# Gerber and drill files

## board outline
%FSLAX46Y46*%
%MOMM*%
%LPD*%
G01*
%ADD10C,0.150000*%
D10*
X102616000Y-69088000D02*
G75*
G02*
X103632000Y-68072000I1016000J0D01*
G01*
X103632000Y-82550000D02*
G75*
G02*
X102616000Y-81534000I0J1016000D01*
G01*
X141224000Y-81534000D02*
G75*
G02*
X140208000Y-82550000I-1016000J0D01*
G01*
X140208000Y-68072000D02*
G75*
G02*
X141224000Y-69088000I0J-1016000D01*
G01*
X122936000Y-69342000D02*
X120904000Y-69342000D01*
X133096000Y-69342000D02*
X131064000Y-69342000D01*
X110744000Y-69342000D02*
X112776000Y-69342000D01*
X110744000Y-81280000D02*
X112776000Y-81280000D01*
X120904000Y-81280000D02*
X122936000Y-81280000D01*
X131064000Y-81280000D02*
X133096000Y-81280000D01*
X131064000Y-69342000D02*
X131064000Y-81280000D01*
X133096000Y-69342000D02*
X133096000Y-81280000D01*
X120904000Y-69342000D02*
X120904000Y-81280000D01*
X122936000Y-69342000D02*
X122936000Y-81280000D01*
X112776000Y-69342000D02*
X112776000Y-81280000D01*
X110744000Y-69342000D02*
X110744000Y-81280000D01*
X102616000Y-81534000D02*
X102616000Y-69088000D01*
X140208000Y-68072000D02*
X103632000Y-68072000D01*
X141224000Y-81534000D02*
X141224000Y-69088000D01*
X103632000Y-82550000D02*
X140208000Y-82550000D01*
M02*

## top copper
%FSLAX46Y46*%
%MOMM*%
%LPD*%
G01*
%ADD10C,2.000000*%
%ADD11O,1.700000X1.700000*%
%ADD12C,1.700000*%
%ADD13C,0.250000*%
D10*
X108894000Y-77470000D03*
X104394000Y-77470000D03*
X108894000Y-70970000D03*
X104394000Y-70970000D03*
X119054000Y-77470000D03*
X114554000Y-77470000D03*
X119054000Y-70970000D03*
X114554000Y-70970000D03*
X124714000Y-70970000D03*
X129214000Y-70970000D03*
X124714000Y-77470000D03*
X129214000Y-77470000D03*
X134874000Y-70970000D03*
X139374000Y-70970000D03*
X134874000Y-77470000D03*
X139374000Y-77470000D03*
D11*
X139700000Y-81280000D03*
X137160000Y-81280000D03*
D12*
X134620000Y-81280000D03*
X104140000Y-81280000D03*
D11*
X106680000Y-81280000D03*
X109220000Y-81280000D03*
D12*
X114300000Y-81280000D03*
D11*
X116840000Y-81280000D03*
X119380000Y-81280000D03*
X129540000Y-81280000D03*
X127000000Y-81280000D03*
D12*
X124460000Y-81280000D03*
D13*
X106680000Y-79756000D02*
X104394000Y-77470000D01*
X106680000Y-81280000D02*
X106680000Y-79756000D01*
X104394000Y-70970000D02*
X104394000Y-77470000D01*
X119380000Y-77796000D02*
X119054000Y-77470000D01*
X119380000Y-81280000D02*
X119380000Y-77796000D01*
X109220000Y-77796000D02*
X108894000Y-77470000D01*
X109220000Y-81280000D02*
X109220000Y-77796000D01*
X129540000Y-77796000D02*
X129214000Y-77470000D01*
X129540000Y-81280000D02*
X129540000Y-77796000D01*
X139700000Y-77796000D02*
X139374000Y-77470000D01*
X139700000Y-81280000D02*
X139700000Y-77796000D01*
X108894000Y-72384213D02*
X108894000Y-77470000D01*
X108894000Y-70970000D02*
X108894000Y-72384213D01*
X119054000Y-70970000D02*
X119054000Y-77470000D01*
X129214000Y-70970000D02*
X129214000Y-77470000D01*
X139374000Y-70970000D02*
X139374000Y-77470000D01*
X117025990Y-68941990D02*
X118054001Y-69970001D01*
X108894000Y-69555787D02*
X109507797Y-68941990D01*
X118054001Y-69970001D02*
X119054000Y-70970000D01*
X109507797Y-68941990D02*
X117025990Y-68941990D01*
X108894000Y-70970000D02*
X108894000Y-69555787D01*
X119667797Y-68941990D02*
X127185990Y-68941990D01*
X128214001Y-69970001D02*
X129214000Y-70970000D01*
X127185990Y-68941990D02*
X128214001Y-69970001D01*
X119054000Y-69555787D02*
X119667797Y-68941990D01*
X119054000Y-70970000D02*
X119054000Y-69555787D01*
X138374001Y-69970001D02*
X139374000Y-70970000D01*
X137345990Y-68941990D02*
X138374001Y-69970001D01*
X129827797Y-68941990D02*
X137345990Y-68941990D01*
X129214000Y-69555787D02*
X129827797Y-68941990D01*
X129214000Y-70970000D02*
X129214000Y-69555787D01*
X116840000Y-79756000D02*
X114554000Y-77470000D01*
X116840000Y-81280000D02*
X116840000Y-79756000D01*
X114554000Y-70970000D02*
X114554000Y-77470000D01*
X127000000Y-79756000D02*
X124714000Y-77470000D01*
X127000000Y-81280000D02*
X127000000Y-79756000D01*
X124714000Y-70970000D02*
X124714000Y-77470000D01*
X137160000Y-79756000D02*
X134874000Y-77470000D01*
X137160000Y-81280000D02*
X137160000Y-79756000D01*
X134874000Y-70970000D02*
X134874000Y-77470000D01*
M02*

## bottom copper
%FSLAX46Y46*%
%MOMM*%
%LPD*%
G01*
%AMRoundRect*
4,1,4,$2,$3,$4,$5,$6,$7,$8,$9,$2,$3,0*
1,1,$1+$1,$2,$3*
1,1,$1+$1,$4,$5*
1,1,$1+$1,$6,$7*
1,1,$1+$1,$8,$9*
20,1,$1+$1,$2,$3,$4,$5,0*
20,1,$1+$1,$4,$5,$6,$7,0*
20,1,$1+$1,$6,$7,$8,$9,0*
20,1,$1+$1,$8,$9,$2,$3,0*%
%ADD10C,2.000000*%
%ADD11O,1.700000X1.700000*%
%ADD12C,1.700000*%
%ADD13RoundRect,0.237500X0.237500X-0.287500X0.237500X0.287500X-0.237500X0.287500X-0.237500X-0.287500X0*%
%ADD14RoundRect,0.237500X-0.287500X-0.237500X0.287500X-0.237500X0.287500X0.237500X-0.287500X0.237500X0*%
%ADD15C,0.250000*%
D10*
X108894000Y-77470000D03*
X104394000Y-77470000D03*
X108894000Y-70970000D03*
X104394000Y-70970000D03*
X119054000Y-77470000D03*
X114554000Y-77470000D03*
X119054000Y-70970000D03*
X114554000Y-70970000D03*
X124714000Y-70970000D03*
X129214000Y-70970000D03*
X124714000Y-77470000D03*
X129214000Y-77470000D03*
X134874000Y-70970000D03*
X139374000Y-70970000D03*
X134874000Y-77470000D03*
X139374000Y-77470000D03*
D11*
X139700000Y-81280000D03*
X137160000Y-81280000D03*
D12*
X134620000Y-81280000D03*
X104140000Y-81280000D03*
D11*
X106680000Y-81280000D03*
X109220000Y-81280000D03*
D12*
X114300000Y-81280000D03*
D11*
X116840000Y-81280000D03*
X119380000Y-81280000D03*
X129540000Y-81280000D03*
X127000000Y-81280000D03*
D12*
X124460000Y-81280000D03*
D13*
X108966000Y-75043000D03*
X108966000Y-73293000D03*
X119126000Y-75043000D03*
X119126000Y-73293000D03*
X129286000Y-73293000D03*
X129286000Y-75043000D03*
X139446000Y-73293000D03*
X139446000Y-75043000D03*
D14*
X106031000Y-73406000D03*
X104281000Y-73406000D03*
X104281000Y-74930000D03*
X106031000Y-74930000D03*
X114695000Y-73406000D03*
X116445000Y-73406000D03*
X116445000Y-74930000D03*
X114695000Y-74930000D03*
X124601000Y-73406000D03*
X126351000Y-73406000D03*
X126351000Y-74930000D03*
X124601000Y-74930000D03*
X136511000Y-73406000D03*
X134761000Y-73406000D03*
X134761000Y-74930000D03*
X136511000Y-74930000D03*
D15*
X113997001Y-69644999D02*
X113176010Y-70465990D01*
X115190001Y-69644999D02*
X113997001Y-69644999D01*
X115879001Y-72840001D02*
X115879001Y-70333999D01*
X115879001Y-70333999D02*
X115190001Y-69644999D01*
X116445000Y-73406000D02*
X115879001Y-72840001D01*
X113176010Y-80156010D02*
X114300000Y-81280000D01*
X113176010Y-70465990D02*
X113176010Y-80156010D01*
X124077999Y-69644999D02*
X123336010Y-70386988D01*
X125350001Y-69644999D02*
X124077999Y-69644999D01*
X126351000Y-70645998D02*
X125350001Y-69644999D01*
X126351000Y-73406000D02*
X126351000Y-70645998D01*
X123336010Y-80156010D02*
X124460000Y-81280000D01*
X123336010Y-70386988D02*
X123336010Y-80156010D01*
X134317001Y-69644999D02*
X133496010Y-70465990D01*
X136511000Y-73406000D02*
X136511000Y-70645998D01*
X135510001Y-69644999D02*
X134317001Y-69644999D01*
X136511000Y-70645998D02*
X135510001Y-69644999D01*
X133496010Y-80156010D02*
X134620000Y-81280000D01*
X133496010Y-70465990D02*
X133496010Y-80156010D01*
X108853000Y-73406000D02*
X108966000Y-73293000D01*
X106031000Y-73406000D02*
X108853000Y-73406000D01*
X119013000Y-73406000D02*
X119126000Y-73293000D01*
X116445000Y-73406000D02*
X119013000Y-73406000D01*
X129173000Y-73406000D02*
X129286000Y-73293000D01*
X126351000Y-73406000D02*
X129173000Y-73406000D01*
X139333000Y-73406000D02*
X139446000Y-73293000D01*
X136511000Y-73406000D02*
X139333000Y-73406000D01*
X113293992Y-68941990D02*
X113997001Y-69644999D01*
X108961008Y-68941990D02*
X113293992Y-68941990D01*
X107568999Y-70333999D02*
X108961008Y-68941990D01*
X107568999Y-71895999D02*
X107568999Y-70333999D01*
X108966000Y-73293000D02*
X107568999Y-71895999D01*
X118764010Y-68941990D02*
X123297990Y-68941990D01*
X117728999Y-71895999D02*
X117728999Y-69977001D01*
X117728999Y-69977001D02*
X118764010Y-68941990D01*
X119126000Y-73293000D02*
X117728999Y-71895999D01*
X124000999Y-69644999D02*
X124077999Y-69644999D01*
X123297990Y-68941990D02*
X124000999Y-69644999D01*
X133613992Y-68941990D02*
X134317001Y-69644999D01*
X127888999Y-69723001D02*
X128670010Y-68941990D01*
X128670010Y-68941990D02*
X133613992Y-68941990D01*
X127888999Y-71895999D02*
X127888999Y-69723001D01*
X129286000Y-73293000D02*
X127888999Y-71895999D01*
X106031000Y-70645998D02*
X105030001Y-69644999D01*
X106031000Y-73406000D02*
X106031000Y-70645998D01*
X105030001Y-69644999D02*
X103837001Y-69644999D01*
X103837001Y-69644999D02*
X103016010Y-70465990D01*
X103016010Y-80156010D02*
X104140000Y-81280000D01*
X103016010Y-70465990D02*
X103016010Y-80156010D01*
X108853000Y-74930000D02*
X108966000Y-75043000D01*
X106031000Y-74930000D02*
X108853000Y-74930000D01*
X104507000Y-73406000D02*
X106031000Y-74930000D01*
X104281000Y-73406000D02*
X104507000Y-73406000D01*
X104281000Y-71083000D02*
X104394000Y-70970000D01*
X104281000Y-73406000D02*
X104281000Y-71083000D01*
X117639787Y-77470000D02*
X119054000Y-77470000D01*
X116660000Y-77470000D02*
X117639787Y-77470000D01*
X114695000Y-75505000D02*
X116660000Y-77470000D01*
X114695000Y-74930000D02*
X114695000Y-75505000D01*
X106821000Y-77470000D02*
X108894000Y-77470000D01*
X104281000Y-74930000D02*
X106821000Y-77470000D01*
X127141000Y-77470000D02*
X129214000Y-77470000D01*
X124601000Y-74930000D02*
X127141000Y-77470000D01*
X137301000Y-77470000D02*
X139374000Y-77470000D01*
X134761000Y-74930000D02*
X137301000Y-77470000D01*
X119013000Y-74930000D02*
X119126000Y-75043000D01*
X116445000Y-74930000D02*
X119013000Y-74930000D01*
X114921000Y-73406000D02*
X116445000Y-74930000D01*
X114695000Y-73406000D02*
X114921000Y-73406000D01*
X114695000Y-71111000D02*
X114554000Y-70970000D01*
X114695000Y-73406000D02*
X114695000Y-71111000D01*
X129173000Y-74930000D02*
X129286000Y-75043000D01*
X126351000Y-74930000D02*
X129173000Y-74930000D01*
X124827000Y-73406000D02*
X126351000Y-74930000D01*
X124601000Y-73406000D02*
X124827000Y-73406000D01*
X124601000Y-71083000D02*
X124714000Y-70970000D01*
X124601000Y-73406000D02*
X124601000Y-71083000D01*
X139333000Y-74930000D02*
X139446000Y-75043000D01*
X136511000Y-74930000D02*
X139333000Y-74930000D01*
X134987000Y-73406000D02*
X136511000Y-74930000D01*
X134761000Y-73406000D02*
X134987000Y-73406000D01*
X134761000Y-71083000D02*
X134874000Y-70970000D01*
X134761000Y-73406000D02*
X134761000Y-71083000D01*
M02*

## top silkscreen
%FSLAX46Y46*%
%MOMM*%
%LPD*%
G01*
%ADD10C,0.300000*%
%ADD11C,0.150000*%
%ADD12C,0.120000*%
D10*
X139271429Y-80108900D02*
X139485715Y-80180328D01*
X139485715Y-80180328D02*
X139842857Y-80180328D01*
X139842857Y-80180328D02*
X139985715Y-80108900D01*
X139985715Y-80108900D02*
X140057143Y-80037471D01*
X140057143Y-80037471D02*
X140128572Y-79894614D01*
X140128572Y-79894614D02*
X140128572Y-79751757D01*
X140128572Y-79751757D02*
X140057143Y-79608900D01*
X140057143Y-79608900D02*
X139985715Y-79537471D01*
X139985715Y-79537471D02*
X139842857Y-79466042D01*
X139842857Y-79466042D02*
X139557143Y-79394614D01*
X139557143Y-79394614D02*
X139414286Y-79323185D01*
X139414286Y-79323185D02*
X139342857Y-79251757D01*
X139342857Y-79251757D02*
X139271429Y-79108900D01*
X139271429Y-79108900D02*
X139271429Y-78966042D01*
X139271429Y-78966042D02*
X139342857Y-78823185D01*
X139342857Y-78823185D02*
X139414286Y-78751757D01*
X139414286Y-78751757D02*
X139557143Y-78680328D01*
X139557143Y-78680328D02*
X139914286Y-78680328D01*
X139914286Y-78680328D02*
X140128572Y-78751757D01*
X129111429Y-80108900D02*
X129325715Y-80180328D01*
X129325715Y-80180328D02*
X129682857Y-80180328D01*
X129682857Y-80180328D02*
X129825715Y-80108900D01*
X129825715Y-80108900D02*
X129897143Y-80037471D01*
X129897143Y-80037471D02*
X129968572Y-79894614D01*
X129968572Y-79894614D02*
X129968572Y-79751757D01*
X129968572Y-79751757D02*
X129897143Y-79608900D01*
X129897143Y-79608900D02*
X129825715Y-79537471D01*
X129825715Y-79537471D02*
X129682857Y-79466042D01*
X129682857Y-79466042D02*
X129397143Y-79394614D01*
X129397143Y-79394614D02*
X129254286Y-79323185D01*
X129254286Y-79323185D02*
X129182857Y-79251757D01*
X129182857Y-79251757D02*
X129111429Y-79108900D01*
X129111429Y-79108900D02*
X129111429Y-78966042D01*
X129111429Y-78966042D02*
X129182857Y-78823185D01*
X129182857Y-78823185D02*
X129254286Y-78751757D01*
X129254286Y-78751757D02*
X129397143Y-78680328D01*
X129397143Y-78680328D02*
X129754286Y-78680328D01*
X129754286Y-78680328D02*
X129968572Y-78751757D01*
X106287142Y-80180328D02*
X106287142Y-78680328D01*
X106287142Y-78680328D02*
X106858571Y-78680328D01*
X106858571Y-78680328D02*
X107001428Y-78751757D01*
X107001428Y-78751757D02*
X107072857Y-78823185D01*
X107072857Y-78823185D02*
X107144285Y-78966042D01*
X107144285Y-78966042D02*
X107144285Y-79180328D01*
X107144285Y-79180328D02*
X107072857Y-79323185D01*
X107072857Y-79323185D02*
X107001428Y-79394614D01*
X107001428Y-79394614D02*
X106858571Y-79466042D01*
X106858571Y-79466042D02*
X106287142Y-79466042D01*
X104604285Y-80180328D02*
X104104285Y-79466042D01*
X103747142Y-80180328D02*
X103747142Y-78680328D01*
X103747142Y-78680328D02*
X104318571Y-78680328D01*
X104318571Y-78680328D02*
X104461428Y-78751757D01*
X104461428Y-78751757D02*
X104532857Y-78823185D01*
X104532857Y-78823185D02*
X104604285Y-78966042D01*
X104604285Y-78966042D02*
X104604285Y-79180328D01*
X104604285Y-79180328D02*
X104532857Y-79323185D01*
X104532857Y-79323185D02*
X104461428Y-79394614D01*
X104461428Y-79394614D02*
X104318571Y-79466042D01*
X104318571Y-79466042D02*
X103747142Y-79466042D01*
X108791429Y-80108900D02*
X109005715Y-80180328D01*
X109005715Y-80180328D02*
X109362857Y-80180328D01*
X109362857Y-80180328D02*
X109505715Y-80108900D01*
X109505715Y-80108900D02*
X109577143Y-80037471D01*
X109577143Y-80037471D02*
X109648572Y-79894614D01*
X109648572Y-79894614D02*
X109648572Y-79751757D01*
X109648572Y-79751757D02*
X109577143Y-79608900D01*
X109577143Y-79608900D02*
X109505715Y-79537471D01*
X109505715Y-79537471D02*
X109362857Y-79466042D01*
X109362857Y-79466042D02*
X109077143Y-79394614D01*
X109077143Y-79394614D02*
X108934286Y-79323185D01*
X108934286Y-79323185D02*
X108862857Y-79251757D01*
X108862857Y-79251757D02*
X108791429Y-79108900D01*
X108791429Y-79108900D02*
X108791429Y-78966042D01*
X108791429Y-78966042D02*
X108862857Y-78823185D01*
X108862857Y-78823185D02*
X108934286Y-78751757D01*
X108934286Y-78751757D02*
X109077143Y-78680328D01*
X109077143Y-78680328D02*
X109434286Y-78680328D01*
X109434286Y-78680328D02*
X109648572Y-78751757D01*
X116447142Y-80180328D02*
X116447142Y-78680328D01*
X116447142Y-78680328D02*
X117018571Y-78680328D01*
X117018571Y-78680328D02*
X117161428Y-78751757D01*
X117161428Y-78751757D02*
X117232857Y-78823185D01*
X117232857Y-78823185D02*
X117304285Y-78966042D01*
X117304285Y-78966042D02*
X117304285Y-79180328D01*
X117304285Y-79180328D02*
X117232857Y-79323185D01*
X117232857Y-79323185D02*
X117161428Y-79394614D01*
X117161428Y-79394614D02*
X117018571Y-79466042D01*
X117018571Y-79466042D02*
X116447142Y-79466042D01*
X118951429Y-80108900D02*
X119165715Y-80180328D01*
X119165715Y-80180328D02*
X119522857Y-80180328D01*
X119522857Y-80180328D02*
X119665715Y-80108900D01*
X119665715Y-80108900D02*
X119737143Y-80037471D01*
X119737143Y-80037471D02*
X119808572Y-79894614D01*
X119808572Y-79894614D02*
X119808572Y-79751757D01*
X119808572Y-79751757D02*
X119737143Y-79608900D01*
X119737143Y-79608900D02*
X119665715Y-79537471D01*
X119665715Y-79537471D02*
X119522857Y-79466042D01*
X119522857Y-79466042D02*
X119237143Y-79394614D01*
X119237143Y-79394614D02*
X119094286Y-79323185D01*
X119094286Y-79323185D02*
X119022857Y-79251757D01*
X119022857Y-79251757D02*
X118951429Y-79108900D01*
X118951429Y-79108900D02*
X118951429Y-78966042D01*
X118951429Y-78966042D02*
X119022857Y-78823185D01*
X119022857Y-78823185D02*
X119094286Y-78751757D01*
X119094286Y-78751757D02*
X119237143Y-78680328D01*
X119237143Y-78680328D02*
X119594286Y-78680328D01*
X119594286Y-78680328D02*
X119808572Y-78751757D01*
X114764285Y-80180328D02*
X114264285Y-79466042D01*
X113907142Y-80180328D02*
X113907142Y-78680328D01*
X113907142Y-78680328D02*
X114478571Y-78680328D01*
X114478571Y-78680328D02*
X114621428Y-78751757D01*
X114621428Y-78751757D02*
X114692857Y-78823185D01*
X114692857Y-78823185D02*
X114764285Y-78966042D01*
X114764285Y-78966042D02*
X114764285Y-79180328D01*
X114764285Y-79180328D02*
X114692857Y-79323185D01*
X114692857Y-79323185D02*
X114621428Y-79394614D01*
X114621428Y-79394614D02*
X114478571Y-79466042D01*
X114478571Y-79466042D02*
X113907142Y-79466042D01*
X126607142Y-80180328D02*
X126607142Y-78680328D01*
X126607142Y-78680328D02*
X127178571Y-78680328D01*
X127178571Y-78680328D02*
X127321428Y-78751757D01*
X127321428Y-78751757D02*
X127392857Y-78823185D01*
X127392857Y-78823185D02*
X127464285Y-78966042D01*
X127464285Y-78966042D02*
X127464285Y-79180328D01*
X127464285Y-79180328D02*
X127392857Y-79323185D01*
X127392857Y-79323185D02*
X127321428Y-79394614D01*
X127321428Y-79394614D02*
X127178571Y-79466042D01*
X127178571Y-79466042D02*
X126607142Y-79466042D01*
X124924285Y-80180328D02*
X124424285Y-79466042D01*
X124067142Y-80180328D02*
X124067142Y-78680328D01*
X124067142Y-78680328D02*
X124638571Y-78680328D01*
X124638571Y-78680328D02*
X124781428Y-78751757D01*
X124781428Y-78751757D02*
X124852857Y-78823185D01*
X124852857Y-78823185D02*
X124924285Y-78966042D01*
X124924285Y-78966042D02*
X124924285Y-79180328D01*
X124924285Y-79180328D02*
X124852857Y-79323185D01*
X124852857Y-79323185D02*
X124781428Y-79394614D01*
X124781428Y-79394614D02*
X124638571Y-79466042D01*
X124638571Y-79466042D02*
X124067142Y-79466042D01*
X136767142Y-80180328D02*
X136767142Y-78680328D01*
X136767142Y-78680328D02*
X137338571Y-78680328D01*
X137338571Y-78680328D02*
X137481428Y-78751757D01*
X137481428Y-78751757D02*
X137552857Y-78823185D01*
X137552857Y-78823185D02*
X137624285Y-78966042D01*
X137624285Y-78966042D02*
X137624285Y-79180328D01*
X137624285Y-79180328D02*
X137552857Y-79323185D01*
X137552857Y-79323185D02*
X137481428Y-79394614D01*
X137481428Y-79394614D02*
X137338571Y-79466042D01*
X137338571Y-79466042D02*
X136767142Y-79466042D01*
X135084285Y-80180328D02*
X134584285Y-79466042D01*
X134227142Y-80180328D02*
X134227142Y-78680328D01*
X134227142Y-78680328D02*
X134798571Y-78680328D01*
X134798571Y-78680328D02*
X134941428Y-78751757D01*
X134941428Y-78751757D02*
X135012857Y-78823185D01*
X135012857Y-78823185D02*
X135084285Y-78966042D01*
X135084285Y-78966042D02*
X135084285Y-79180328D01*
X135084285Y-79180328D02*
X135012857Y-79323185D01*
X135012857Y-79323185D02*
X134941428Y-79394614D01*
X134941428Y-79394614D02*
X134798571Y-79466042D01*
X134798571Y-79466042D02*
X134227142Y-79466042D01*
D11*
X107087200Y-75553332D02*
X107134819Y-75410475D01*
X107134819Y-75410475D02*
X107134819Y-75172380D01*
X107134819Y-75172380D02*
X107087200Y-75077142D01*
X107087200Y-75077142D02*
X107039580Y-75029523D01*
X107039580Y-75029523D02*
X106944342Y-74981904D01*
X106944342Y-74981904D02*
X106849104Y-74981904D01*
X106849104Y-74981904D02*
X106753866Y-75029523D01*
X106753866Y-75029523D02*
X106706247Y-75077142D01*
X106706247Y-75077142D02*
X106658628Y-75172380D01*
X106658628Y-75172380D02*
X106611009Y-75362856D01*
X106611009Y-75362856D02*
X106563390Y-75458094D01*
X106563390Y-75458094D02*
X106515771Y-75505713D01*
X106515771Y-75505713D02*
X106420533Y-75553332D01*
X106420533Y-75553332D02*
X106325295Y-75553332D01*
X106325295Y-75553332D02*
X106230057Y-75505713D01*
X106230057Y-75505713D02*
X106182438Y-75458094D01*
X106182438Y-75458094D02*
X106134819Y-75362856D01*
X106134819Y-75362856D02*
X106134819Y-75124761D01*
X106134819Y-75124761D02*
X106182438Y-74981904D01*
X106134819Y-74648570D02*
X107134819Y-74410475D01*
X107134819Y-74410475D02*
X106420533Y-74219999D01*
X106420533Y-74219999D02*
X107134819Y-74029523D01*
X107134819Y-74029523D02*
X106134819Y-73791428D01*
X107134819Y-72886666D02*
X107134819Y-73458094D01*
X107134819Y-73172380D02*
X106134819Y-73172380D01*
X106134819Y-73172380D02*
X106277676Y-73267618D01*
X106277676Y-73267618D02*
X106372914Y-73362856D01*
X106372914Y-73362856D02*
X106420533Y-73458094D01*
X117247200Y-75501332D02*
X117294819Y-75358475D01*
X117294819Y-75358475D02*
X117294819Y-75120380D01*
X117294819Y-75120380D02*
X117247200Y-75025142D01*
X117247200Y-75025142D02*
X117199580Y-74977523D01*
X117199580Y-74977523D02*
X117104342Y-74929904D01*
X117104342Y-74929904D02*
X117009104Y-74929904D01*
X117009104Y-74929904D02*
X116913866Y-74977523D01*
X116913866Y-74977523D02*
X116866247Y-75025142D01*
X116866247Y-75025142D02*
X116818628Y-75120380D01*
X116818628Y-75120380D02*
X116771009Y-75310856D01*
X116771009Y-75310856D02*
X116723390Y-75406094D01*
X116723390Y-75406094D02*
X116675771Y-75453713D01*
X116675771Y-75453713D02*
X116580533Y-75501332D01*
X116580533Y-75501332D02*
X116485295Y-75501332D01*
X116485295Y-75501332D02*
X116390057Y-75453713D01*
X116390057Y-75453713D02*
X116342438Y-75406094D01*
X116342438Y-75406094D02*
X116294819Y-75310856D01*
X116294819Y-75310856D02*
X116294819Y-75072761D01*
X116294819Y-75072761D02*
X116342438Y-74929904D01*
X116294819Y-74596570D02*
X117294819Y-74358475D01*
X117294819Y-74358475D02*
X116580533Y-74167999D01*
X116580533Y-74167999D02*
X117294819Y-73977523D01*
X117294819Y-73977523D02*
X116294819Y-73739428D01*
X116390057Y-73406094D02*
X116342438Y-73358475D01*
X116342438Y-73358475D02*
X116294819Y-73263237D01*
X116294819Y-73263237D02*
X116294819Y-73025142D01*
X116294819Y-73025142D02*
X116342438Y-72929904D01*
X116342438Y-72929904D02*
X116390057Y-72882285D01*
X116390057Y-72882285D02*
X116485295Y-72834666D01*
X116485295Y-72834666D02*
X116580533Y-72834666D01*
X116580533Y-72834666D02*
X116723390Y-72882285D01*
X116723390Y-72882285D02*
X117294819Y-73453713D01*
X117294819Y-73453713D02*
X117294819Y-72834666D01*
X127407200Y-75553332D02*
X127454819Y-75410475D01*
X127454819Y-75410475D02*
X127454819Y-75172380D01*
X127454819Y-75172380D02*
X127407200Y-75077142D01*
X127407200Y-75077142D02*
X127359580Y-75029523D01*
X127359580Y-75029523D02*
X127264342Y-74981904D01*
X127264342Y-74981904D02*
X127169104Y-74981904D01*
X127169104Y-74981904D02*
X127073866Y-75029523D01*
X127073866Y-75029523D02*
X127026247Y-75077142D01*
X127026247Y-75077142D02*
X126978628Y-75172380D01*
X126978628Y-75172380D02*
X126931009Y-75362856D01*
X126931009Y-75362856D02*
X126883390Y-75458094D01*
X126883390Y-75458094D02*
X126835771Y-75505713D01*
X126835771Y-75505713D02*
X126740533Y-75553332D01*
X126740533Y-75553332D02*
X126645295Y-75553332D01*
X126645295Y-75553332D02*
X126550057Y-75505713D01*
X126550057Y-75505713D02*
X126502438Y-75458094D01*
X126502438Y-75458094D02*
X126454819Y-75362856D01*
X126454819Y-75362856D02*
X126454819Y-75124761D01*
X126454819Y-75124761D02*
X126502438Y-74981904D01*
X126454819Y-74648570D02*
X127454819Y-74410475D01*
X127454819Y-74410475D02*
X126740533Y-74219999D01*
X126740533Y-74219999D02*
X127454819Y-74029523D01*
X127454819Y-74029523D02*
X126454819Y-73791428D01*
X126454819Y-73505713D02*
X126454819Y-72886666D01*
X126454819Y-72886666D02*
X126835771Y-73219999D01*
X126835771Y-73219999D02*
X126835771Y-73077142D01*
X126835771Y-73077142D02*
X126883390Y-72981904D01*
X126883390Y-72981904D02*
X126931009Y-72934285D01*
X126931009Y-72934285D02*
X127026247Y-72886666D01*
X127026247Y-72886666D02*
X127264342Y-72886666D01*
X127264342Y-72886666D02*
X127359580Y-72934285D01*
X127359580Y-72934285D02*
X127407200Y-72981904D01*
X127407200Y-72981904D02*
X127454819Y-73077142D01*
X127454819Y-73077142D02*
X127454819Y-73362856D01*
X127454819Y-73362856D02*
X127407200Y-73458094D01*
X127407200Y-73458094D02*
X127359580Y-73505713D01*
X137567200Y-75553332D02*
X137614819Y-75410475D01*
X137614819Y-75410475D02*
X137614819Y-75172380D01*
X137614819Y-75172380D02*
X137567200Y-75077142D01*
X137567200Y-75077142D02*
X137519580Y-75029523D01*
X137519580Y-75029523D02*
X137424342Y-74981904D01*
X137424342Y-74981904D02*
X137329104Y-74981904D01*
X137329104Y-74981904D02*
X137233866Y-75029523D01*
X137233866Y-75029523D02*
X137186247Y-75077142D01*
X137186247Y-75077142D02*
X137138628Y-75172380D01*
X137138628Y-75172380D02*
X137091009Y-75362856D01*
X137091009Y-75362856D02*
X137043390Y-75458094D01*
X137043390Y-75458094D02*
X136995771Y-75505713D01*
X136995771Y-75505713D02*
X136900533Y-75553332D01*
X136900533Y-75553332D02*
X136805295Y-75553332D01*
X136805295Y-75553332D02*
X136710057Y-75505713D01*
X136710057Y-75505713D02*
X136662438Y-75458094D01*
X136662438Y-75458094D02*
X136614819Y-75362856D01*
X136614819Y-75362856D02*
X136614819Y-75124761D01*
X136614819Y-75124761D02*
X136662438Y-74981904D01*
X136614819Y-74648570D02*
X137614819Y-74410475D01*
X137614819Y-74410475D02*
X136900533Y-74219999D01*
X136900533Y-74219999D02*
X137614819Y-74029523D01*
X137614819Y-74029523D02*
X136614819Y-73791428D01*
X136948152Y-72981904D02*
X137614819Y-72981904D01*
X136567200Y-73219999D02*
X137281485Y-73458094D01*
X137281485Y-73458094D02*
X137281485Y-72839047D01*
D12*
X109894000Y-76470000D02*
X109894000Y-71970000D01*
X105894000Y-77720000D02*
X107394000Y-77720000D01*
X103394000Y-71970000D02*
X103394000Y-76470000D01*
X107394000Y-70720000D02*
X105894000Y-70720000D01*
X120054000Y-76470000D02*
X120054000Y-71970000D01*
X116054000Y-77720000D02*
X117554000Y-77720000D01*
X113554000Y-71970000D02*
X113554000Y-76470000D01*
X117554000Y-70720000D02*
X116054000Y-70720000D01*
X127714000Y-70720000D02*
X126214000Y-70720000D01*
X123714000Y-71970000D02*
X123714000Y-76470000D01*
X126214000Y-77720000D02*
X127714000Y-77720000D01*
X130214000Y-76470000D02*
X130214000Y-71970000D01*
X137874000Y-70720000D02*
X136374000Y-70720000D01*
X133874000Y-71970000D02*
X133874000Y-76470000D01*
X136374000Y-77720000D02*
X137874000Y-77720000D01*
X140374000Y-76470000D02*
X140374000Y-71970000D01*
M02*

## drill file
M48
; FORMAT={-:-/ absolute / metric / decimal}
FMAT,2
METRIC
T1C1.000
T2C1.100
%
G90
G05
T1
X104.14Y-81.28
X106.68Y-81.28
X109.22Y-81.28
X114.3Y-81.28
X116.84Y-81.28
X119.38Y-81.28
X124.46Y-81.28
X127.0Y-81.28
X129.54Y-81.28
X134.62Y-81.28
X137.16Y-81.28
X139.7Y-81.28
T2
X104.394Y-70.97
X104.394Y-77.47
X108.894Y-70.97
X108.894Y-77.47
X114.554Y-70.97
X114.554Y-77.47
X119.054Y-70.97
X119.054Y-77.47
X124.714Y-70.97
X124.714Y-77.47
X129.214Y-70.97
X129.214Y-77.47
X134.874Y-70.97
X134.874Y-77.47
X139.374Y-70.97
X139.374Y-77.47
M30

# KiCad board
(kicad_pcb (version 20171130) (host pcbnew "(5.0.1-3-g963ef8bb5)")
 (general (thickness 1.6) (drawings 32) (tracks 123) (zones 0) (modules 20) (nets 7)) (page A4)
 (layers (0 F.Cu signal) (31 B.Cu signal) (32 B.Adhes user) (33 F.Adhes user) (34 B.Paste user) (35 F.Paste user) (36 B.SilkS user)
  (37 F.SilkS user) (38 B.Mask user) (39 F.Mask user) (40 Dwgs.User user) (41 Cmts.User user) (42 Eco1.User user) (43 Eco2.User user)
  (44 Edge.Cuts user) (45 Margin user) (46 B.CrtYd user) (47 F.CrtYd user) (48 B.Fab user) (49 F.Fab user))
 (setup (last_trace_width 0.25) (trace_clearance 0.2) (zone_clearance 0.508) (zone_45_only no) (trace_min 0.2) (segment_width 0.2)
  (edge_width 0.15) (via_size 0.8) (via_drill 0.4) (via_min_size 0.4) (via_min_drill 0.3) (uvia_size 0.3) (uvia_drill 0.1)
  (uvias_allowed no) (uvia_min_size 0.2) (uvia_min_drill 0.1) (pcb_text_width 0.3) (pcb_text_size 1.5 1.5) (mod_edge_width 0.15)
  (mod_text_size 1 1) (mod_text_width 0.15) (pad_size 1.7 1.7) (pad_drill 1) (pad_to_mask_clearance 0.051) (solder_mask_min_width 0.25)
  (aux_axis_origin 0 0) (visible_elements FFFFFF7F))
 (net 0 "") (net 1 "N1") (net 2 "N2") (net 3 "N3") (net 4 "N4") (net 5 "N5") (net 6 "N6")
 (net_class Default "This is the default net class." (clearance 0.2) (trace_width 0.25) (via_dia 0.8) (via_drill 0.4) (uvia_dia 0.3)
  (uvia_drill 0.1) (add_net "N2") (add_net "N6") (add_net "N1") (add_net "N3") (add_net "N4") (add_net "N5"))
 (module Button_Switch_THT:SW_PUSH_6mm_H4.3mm (layer F.Cu) (at 104.394 77.47 90)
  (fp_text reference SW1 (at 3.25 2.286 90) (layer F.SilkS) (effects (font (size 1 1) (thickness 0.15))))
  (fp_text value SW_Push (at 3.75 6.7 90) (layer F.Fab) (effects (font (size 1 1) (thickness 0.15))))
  (fp_line (start 1 5.5) (end 5.5 5.5) (layer F.SilkS) (width 0.12))
  (fp_line (start -0.25 1.5) (end -0.25 3) (layer F.SilkS) (width 0.12))
  (fp_line (start 5.5 -1) (end 1 -1) (layer F.SilkS) (width 0.12))
  (fp_line (start 6.75 3) (end 6.75 1.5) (layer F.SilkS) (width 0.12))
  (pad 2 thru_hole circle (at 0 4.5 180) (size 2 2) (drill 1.1) (layers *.Cu *.Mask) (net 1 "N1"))
  (pad 1 thru_hole circle (at 0 0 180) (size 2 2) (drill 1.1) (layers *.Cu *.Mask) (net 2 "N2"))
  (pad 2 thru_hole circle (at 6.5 4.5 180) (size 2 2) (drill 1.1) (layers *.Cu *.Mask) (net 1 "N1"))
  (pad 1 thru_hole circle (at 6.5 0 180) (size 2 2) (drill 1.1) (layers *.Cu *.Mask) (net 2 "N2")))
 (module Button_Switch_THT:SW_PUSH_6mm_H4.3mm (layer F.Cu) (at 114.554 77.47 90)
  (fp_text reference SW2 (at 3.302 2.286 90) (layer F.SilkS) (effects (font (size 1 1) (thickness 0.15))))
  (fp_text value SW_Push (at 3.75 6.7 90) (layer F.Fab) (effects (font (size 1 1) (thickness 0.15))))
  (fp_line (start 1 5.5) (end 5.5 5.5) (layer F.SilkS) (width 0.12))
  (fp_line (start -0.25 1.5) (end -0.25 3) (layer F.SilkS) (width 0.12))
  (fp_line (start 5.5 -1) (end 1 -1) (layer F.SilkS) (width 0.12))
  (fp_line (start 6.75 3) (end 6.75 1.5) (layer F.SilkS) (width 0.12))
  (pad 2 thru_hole circle (at 0 4.5 180) (size 2 2) (drill 1.1) (layers *.Cu *.Mask) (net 1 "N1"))
  (pad 1 thru_hole circle (at 0 0 180) (size 2 2) (drill 1.1) (layers *.Cu *.Mask) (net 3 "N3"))
  (pad 2 thru_hole circle (at 6.5 4.5 180) (size 2 2) (drill 1.1) (layers *.Cu *.Mask) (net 1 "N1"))
  (pad 1 thru_hole circle (at 6.5 0 180) (size 2 2) (drill 1.1) (layers *.Cu *.Mask) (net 3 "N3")))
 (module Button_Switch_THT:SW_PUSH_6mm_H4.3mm (layer F.Cu) (at 124.714 77.47 90)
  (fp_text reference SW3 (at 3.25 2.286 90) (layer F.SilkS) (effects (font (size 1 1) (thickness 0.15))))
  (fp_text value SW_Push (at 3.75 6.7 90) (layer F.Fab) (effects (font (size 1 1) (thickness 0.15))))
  (fp_line (start 6.75 3) (end 6.75 1.5) (layer F.SilkS) (width 0.12))
  (fp_line (start 5.5 -1) (end 1 -1) (layer F.SilkS) (width 0.12))
  (fp_line (start -0.25 1.5) (end -0.25 3) (layer F.SilkS) (width 0.12))
  (fp_line (start 1 5.5) (end 5.5 5.5) (layer F.SilkS) (width 0.12))
  (pad 1 thru_hole circle (at 6.5 0 180) (size 2 2) (drill 1.1) (layers *.Cu *.Mask) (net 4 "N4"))
  (pad 2 thru_hole circle (at 6.5 4.5 180) (size 2 2) (drill 1.1) (layers *.Cu *.Mask) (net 1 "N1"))
  (pad 1 thru_hole circle (at 0 0 180) (size 2 2) (drill 1.1) (layers *.Cu *.Mask) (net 4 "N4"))
  (pad 2 thru_hole circle (at 0 4.5 180) (size 2 2) (drill 1.1) (layers *.Cu *.Mask) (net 1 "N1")))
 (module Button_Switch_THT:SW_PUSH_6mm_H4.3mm (layer F.Cu) (at 134.874 77.47 90)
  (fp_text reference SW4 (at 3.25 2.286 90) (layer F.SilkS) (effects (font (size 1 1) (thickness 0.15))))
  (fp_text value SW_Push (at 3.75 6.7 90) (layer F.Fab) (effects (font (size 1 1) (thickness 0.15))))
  (fp_line (start 6.75 3) (end 6.75 1.5) (layer F.SilkS) (width 0.12))
  (fp_line (start 5.5 -1) (end 1 -1) (layer F.SilkS) (width 0.12))
  (fp_line (start -0.25 1.5) (end -0.25 3) (layer F.SilkS) (width 0.12))
  (fp_line (start 1 5.5) (end 5.5 5.5) (layer F.SilkS) (width 0.12))
  (pad 1 thru_hole circle (at 6.5 0 180) (size 2 2) (drill 1.1) (layers *.Cu *.Mask) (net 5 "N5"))
  (pad 2 thru_hole circle (at 6.5 4.5 180) (size 2 2) (drill 1.1) (layers *.Cu *.Mask) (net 1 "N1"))
  (pad 1 thru_hole circle (at 0 0 180) (size 2 2) (drill 1.1) (layers *.Cu *.Mask) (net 5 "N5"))
  (pad 2 thru_hole circle (at 0 4.5 180) (size 2 2) (drill 1.1) (layers *.Cu *.Mask) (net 1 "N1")))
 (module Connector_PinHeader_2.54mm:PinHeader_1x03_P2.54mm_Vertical (layer B.Cu) (at 134.62 81.28 270)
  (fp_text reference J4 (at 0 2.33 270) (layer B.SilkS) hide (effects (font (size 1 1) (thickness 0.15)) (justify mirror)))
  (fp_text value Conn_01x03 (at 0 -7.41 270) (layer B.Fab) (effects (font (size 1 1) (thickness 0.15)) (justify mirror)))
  (pad 3 thru_hole oval (at 0 -5.08 270) (size 1.7 1.7) (drill 1) (layers *.Cu *.Mask) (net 1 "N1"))
  (pad 2 thru_hole oval (at 0 -2.54 270) (size 1.7 1.7) (drill 1) (layers *.Cu *.Mask) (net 5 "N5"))
  (pad 1 thru_hole circle (at 0 0 270) (size 1.7 1.7) (drill 1) (layers *.Cu *.Mask) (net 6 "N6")))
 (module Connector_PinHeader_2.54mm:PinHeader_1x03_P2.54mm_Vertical (layer B.Cu) (at 104.14 81.28 270)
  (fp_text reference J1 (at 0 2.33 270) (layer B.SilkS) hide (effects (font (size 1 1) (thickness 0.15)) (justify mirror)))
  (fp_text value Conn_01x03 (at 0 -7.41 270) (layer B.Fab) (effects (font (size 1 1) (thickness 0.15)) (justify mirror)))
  (pad 1 thru_hole circle (at 0 0 270) (size 1.7 1.7) (drill 1) (layers *.Cu *.Mask) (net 6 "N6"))
  (pad 2 thru_hole oval (at 0 -2.54 270) (size 1.7 1.7) (drill 1) (layers *.Cu *.Mask) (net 2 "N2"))
  (pad 3 thru_hole oval (at 0 -5.08 270) (size 1.7 1.7) (drill 1) (layers *.Cu *.Mask) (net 1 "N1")))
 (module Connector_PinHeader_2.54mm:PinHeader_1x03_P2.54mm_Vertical (layer B.Cu) (at 114.3 81.28 270)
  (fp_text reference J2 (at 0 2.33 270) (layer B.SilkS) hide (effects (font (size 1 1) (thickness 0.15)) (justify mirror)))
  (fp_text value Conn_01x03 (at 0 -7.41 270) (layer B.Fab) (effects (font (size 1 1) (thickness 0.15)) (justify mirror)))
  (pad 1 thru_hole circle (at 0 0 270) (size 1.7 1.7) (drill 1) (layers *.Cu *.Mask) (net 6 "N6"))
  (pad 2 thru_hole oval (at 0 -2.54 270) (size 1.7 1.7) (drill 1) (layers *.Cu *.Mask) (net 3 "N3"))
  (pad 3 thru_hole oval (at 0 -5.08 270) (size 1.7 1.7) (drill 1) (layers *.Cu *.Mask) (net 1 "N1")))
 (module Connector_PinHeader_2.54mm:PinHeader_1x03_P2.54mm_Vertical (layer B.Cu) (at 124.46 81.28 270)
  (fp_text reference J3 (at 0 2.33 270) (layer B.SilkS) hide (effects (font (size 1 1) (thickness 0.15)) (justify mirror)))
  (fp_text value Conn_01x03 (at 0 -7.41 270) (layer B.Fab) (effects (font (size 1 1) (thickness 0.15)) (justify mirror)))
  (pad 3 thru_hole oval (at 0 -5.08 270) (size 1.7 1.7) (drill 1) (layers *.Cu *.Mask) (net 1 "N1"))
  (pad 2 thru_hole oval (at 0 -2.54 270) (size 1.7 1.7) (drill 1) (layers *.Cu *.Mask) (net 4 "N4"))
  (pad 1 thru_hole circle (at 0 0 270) (size 1.7 1.7) (drill 1) (layers *.Cu *.Mask) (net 6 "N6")))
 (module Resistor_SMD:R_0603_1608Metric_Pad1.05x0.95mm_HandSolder (layer B.Cu) (at 108.966 74.168 90)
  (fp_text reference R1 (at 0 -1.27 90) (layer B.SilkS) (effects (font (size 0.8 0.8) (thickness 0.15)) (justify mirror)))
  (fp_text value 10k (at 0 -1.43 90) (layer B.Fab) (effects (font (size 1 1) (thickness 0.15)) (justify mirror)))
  (pad 1 smd roundrect (at -0.875 0 90) (size 1.05 0.95) (layers B.Cu B.Paste B.Mask) (roundrect_rratio 0.25) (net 2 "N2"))
  (pad 2 smd roundrect (at 0.875 0 90) (size 1.05 0.95) (layers B.Cu B.Paste B.Mask) (roundrect_rratio 0.25) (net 6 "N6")))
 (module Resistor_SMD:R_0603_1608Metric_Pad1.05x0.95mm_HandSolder (layer B.Cu) (at 119.126 74.168 90)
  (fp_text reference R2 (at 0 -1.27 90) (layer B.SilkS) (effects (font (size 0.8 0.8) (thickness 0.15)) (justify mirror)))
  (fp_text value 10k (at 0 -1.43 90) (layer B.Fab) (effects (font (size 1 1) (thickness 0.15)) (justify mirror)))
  (pad 1 smd roundrect (at -0.875 0 90) (size 1.05 0.95) (layers B.Cu B.Paste B.Mask) (roundrect_rratio 0.25) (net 3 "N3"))
  (pad 2 smd roundrect (at 0.875 0 90) (size 1.05 0.95) (layers B.Cu B.Paste B.Mask) (roundrect_rratio 0.25) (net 6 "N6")))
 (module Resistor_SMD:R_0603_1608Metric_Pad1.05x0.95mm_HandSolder (layer B.Cu) (at 129.286 74.168 90)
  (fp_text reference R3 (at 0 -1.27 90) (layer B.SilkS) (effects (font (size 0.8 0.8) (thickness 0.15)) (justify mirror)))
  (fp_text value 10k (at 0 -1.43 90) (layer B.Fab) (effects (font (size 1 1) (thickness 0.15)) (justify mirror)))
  (pad 2 smd roundrect (at 0.875 0 90) (size 1.05 0.95) (layers B.Cu B.Paste B.Mask) (roundrect_rratio 0.25) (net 6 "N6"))
  (pad 1 smd roundrect (at -0.875 0 90) (size 1.05 0.95) (layers B.Cu B.Paste B.Mask) (roundrect_rratio 0.25) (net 4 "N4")))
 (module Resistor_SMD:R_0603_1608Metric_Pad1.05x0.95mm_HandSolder (layer B.Cu) (at 139.446 74.168 90)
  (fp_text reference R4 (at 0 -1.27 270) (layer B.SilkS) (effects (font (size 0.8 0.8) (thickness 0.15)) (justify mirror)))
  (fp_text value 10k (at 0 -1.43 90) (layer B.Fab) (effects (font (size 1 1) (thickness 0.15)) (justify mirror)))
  (pad 2 smd roundrect (at 0.875 0 90) (size 1.05 0.95) (layers B.Cu B.Paste B.Mask) (roundrect_rratio 0.25) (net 6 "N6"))
  (pad 1 smd roundrect (at -0.875 0 90) (size 1.05 0.95) (layers B.Cu B.Paste B.Mask) (roundrect_rratio 0.25) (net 5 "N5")))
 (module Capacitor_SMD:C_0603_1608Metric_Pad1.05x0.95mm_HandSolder (layer B.Cu) (at 105.156 73.406)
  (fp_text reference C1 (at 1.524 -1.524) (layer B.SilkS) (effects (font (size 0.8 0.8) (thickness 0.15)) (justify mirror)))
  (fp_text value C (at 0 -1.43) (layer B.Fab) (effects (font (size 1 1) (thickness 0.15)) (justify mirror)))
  (pad 2 smd roundrect (at 0.875 0) (size 1.05 0.95) (layers B.Cu B.Paste B.Mask) (roundrect_rratio 0.25) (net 6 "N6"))
  (pad 1 smd roundrect (at -0.875 0) (size 1.05 0.95) (layers B.Cu B.Paste B.Mask) (roundrect_rratio 0.25) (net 2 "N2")))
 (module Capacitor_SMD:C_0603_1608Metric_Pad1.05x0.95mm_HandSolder (layer B.Cu) (at 105.156 74.93)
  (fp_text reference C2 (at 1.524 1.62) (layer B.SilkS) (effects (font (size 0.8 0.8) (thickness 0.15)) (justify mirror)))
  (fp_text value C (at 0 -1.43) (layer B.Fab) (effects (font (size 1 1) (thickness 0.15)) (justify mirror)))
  (pad 1 smd roundrect (at -0.875 0) (size 1.05 0.95) (layers B.Cu B.Paste B.Mask) (roundrect_rratio 0.25) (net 1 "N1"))
  (pad 2 smd roundrect (at 0.875 0) (size 1.05 0.95) (layers B.Cu B.Paste B.Mask) (roundrect_rratio 0.25) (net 2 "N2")))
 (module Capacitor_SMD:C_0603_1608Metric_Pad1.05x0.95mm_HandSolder (layer B.Cu) (at 115.57 73.406)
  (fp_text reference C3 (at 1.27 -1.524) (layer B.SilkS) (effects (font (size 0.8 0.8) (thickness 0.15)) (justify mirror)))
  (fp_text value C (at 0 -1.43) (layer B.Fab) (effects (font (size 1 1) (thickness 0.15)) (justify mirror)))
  (pad 1 smd roundrect (at -0.875 0) (size 1.05 0.95) (layers B.Cu B.Paste B.Mask) (roundrect_rratio 0.25) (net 3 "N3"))
  (pad 2 smd roundrect (at 0.875 0) (size 1.05 0.95) (layers B.Cu B.Paste B.Mask) (roundrect_rratio 0.25) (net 6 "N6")))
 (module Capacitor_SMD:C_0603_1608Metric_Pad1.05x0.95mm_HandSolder (layer B.Cu) (at 115.57 74.93)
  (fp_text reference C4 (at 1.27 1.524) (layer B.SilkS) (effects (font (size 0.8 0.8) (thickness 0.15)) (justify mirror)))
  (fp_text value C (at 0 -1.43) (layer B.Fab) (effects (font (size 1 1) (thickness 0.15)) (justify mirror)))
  (pad 2 smd roundrect (at 0.875 0) (size 1.05 0.95) (layers B.Cu B.Paste B.Mask) (roundrect_rratio 0.25) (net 3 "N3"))
  (pad 1 smd roundrect (at -0.875 0) (size 1.05 0.95) (layers B.Cu B.Paste B.Mask) (roundrect_rratio 0.25) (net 1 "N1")))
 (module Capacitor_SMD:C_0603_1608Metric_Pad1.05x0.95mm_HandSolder (layer B.Cu) (at 125.476 73.406)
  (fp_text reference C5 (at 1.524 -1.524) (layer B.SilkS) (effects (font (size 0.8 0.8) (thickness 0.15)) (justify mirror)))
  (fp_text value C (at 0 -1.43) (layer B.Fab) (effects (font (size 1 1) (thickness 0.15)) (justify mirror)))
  (pad 1 smd roundrect (at -0.875 0) (size 1.05 0.95) (layers B.Cu B.Paste B.Mask) (roundrect_rratio 0.25) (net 4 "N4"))
  (pad 2 smd roundrect (at 0.875 0) (size 1.05 0.95) (layers B.Cu B.Paste B.Mask) (roundrect_rratio 0.25) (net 6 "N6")))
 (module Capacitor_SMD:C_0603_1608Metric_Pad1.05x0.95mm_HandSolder (layer B.Cu) (at 125.476 74.93)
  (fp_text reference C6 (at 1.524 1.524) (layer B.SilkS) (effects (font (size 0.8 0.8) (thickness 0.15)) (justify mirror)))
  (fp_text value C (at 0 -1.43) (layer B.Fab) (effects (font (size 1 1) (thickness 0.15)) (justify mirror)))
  (pad 2 smd roundrect (at 0.875 0) (size 1.05 0.95) (layers B.Cu B.Paste B.Mask) (roundrect_rratio 0.25) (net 4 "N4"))
  (pad 1 smd roundrect (at -0.875 0) (size 1.05 0.95) (layers B.Cu B.Paste B.Mask) (roundrect_rratio 0.25) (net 1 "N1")))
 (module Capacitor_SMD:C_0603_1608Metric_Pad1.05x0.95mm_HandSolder (layer B.Cu) (at 135.636 73.406)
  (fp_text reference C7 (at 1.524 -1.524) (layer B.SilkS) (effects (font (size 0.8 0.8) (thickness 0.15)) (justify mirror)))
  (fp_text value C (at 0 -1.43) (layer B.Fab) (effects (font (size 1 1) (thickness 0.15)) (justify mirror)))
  (pad 2 smd roundrect (at 0.875 0) (size 1.05 0.95) (layers B.Cu B.Paste B.Mask) (roundrect_rratio 0.25) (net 6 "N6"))
  (pad 1 smd roundrect (at -0.875 0) (size 1.05 0.95) (layers B.Cu B.Paste B.Mask) (roundrect_rratio 0.25) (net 5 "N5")))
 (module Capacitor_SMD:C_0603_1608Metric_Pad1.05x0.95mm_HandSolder (layer B.Cu) (at 135.636 74.93)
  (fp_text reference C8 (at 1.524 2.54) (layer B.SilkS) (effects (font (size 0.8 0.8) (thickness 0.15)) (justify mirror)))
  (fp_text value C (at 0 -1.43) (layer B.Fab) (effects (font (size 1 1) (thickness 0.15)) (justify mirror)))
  (pad 1 smd roundrect (at -0.875 0) (size 1.05 0.95) (layers B.Cu B.Paste B.Mask) (roundrect_rratio 0.25) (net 1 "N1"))
  (pad 2 smd roundrect (at 0.875 0) (size 1.05 0.95) (layers B.Cu B.Paste B.Mask) (roundrect_rratio 0.25) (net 5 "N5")))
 (gr_arc (start 103.632 69.088) (end 103.632 68.072) (angle -90) (layer Edge.Cuts) (width 0.15))
 (gr_arc (start 103.632 81.534) (end 102.616 81.534) (angle -90) (layer Edge.Cuts) (width 0.15))
 (gr_arc (start 140.208 81.534) (end 140.208 82.55) (angle -90) (layer Edge.Cuts) (width 0.15))
 (gr_arc (start 140.208 69.088) (end 141.224 69.088) (angle -90) (layer Edge.Cuts) (width 0.15))
 (gr_line (start 122.936 69.342) (end 120.904 69.342) (layer Edge.Cuts) (width 0.15))
 (gr_line (start 133.096 69.342) (end 131.064 69.342) (layer Edge.Cuts) (width 0.15))
 (gr_line (start 110.744 69.342) (end 112.776 69.342) (layer Edge.Cuts) (width 0.15))
 (gr_line (start 110.744 81.28) (end 112.776 81.28) (layer Edge.Cuts) (width 0.15))
 (gr_line (start 120.904 81.28) (end 122.936 81.28) (layer Edge.Cuts) (width 0.15))
 (gr_line (start 131.064 81.28) (end 133.096 81.28) (layer Edge.Cuts) (width 0.15))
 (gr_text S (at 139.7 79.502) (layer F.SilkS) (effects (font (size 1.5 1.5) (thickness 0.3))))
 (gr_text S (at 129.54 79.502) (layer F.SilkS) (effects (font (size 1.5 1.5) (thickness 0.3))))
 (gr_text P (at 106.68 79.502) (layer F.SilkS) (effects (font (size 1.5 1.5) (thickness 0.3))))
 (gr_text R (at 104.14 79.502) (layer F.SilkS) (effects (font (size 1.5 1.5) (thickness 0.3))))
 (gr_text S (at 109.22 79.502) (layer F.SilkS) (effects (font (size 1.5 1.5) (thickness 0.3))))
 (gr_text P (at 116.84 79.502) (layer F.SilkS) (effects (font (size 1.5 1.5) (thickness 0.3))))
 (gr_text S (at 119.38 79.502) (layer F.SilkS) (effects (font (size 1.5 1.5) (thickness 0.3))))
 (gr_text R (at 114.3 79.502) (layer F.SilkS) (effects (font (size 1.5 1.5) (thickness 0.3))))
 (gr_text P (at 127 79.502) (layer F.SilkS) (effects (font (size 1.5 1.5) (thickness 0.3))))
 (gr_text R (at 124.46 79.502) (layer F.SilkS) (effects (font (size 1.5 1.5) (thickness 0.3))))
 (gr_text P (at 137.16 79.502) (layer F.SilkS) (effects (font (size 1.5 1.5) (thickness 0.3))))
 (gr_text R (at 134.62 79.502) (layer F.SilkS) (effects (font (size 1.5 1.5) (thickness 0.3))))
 (gr_line (start 131.064 69.342) (end 131.064 81.28) (layer Edge.Cuts) (width 0.15))
 (gr_line (start 133.096 69.342) (end 133.096 81.28) (layer Edge.Cuts) (width 0.15))
 (gr_line (start 120.904 69.342) (end 120.904 81.28) (layer Edge.Cuts) (width 0.15))
 (gr_line (start 122.936 69.342) (end 122.936 81.28) (layer Edge.Cuts) (width 0.15))
 (gr_line (start 112.776 69.342) (end 112.776 81.28) (layer Edge.Cuts) (width 0.15))
 (gr_line (start 110.744 69.342) (end 110.744 81.28) (layer Edge.Cuts) (width 0.15))
 (gr_line (start 102.616 81.534) (end 102.616 69.088) (layer Edge.Cuts) (width 0.15))
 (gr_line (start 140.208 68.072) (end 103.632 68.072) (layer Edge.Cuts) (width 0.15))
 (gr_line (start 141.224 81.534) (end 141.224 69.088) (layer Edge.Cuts) (width 0.15))
 (gr_line (start 103.632 82.55) (end 140.208 82.55) (layer Edge.Cuts) (width 0.15))
 (segment (start 113.997001 69.644999) (end 113.17601 70.46599) (width 0.25) (layer B.Cu) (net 6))
 (segment (start 115.190001 69.644999) (end 113.997001 69.644999) (width 0.25) (layer B.Cu) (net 6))
 (segment (start 115.879001 72.840001) (end 115.879001 70.333999) (width 0.25) (layer B.Cu) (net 6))
 (segment (start 115.879001 70.333999) (end 115.190001 69.644999) (width 0.25) (layer B.Cu) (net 6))
 (segment (start 116.445 73.406) (end 115.879001 72.840001) (width 0.25) (layer B.Cu) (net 6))
 (segment (start 113.17601 80.15601) (end 114.3 81.28) (width 0.25) (layer B.Cu) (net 6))
 (segment (start 113.17601 70.46599) (end 113.17601 80.15601) (width 0.25) (layer B.Cu) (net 6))
 (segment (start 124.077999 69.644999) (end 123.33601 70.386988) (width 0.25) (layer B.Cu) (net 6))
 (segment (start 125.350001 69.644999) (end 124.077999 69.644999) (width 0.25) (layer B.Cu) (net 6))
 (segment (start 126.351 70.645998) (end 125.350001 69.644999) (width 0.25) (layer B.Cu) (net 6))
 (segment (start 126.351 73.406) (end 126.351 70.645998) (width 0.25) (layer B.Cu) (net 6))
 (segment (start 123.33601 80.15601) (end 124.46 81.28) (width 0.25) (layer B.Cu) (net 6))
 (segment (start 123.33601 70.386988) (end 123.33601 80.15601) (width 0.25) (layer B.Cu) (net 6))
 (segment (start 134.317001 69.644999) (end 133.49601 70.46599) (width 0.25) (layer B.Cu) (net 6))
 (segment (start 136.511 73.406) (end 136.511 70.645998) (width 0.25) (layer B.Cu) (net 6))
 (segment (start 135.510001 69.644999) (end 134.317001 69.644999) (width 0.25) (layer B.Cu) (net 6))
 (segment (start 136.511 70.645998) (end 135.510001 69.644999) (width 0.25) (layer B.Cu) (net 6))
 (segment (start 133.49601 80.15601) (end 134.62 81.28) (width 0.25) (layer B.Cu) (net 6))
 (segment (start 133.49601 70.46599) (end 133.49601 80.15601) (width 0.25) (layer B.Cu) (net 6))
 (segment (start 108.853 73.406) (end 108.966 73.293) (width 0.25) (layer B.Cu) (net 6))
 (segment (start 106.031 73.406) (end 108.853 73.406) (width 0.25) (layer B.Cu) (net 6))
 (segment (start 119.013 73.406) (end 119.126 73.293) (width 0.25) (layer B.Cu) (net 6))
 (segment (start 116.445 73.406) (end 119.013 73.406) (width 0.25) (layer B.Cu) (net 6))
 (segment (start 129.173 73.406) (end 129.286 73.293) (width 0.25) (layer B.Cu) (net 6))
 (segment (start 126.351 73.406) (end 129.173 73.406) (width 0.25) (layer B.Cu) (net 6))
 (segment (start 139.333 73.406) (end 139.446 73.293) (width 0.25) (layer B.Cu) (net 6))
 (segment (start 136.511 73.406) (end 139.333 73.406) (width 0.25) (layer B.Cu) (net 6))
 (segment (start 113.293992 68.94199) (end 113.997001 69.644999) (width 0.25) (layer B.Cu) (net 6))
 (segment (start 108.961008 68.94199) (end 113.293992 68.94199) (width 0.25) (layer B.Cu) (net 6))
 (segment (start 107.568999 70.333999) (end 108.961008 68.94199) (width 0.25) (layer B.Cu) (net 6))
 (segment (start 107.568999 71.895999) (end 107.568999 70.333999) (width 0.25) (layer B.Cu) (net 6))
 (segment (start 108.966 73.293) (end 107.568999 71.895999) (width 0.25) (layer B.Cu) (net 6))
 (segment (start 118.76401 68.94199) (end 123.29799 68.94199) (width 0.25) (layer B.Cu) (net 6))
 (segment (start 117.728999 71.895999) (end 117.728999 69.977001) (width 0.25) (layer B.Cu) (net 6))
 (segment (start 117.728999 69.977001) (end 118.76401 68.94199) (width 0.25) (layer B.Cu) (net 6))
 (segment (start 119.126 73.293) (end 117.728999 71.895999) (width 0.25) (layer B.Cu) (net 6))
 (segment (start 124.000999 69.644999) (end 124.077999 69.644999) (width 0.25) (layer B.Cu) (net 6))
 (segment (start 123.29799 68.94199) (end 124.000999 69.644999) (width 0.25) (layer B.Cu) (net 6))
 (segment (start 133.613992 68.94199) (end 134.317001 69.644999) (width 0.25) (layer B.Cu) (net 6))
 (segment (start 127.888999 69.723001) (end 128.67001 68.94199) (width 0.25) (layer B.Cu) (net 6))
 (segment (start 128.67001 68.94199) (end 133.613992 68.94199) (width 0.25) (layer B.Cu) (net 6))
 (segment (start 127.888999 71.895999) (end 127.888999 69.723001) (width 0.25) (layer B.Cu) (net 6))
 (segment (start 129.286 73.293) (end 127.888999 71.895999) (width 0.25) (layer B.Cu) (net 6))
 (segment (start 106.031 70.645998) (end 105.030001 69.644999) (width 0.25) (layer B.Cu) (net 6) (status 1000000))
 (segment (start 106.031 73.406) (end 106.031 70.645998) (width 0.25) (layer B.Cu) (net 6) (status 1000000))
 (segment (start 105.030001 69.644999) (end 103.837001 69.644999) (width 0.25) (layer B.Cu) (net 6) (status 1000000))
 (segment (start 103.837001 69.644999) (end 103.01601 70.46599) (width 0.25) (layer B.Cu) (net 6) (status 1000000))
 (segment (start 103.01601 80.15601) (end 104.14 81.28) (width 0.25) (layer B.Cu) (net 6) (status 1000000))
 (segment (start 103.01601 70.46599) (end 103.01601 80.15601) (width 0.25) (layer B.Cu) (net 6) (status 1000000))
 (segment (start 106.68 79.756) (end 104.394 77.47) (width 0.25) (layer F.Cu) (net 2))
 (segment (start 106.68 81.28) (end 106.68 79.756) (width 0.25) (layer F.Cu) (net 2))
 (segment (start 104.394 70.97) (end 104.394 77.47) (width 0.25) (layer F.Cu) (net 2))
 (segment (start 108.853 74.93) (end 108.966 75.043) (width 0.25) (layer B.Cu) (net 2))
 (segment (start 106.031 74.93) (end 108.853 74.93) (width 0.25) (layer B.Cu) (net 2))
 (segment (start 104.507 73.406) (end 106.031 74.93) (width 0.25) (layer B.Cu) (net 2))
 (segment (start 104.281 73.406) (end 104.507 73.406) (width 0.25) (layer B.Cu) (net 2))
 (segment (start 104.281 71.083) (end 104.394 70.97) (width 0.25) (layer B.Cu) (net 2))
 (segment (start 104.281 73.406) (end 104.281 71.083) (width 0.25) (layer B.Cu) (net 2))
 (segment (start 119.38 77.796) (end 119.054 77.47) (width 0.25) (layer F.Cu) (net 1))
 (segment (start 119.38 81.28) (end 119.38 77.796) (width 0.25) (layer F.Cu) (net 1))
 (segment (start 109.22 77.796) (end 108.894 77.47) (width 0.25) (layer F.Cu) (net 1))
 (segment (start 109.22 81.28) (end 109.22 77.796) (width 0.25) (layer F.Cu) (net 1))
 (segment (start 129.54 77.796) (end 129.214 77.47) (width 0.25) (layer F.Cu) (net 1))
 (segment (start 129.54 81.28) (end 129.54 77.796) (width 0.25) (layer F.Cu) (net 1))
 (segment (start 139.7 77.796) (end 139.374 77.47) (width 0.25) (layer F.Cu) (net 1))
 (segment (start 139.7 81.28) (end 139.7 77.796) (width 0.25) (layer F.Cu) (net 1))
 (segment (start 108.894 72.384213) (end 108.894 77.47) (width 0.25) (layer F.Cu) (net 1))
 (segment (start 108.894 70.97) (end 108.894 72.384213) (width 0.25) (layer F.Cu) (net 1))
 (segment (start 119.054 70.97) (end 119.054 77.47) (width 0.25) (layer F.Cu) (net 1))
 (segment (start 129.214 70.97) (end 129.214 77.47) (width 0.25) (layer F.Cu) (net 1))
 (segment (start 139.374 70.97) (end 139.374 77.47) (width 0.25) (layer F.Cu) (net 1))
 (segment (start 117.639787 77.47) (end 119.054 77.47) (width 0.25) (layer B.Cu) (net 1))
 (segment (start 116.66 77.47) (end 117.639787 77.47) (width 0.25) (layer B.Cu) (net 1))
 (segment (start 114.695 75.505) (end 116.66 77.47) (width 0.25) (layer B.Cu) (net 1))
 (segment (start 114.695 74.93) (end 114.695 75.505) (width 0.25) (layer B.Cu) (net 1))
 (segment (start 106.821 77.47) (end 108.894 77.47) (width 0.25) (layer B.Cu) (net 1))
 (segment (start 104.281 74.93) (end 106.821 77.47) (width 0.25) (layer B.Cu) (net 1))
 (segment (start 127.141 77.47) (end 129.214 77.47) (width 0.25) (layer B.Cu) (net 1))
 (segment (start 124.601 74.93) (end 127.141 77.47) (width 0.25) (layer B.Cu) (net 1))
 (segment (start 137.301 77.47) (end 139.374 77.47) (width 0.25) (layer B.Cu) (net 1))
 (segment (start 134.761 74.93) (end 137.301 77.47) (width 0.25) (layer B.Cu) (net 1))
 (segment (start 117.02599 68.94199) (end 118.054001 69.970001) (width 0.25) (layer F.Cu) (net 1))
 (segment (start 108.894 69.555787) (end 109.507797 68.94199) (width 0.25) (layer F.Cu) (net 1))
 (segment (start 118.054001 69.970001) (end 119.054 70.97) (width 0.25) (layer F.Cu) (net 1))
 (segment (start 109.507797 68.94199) (end 117.02599 68.94199) (width 0.25) (layer F.Cu) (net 1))
 (segment (start 108.894 70.97) (end 108.894 69.555787) (width 0.25) (layer F.Cu) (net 1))
 (segment (start 119.667797 68.94199) (end 127.18599 68.94199) (width 0.25) (layer F.Cu) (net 1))
 (segment (start 128.214001 69.970001) (end 129.214 70.97) (width 0.25) (layer F.Cu) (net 1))
 (segment (start 127.18599 68.94199) (end 128.214001 69.970001) (width 0.25) (layer F.Cu) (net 1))
 (segment (start 119.054 69.555787) (end 119.667797 68.94199) (width 0.25) (layer F.Cu) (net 1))
 (segment (start 119.054 70.97) (end 119.054 69.555787) (width 0.25) (layer F.Cu) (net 1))
 (segment (start 138.374001 69.970001) (end 139.374 70.97) (width 0.25) (layer F.Cu) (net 1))
 (segment (start 137.34599 68.94199) (end 138.374001 69.970001) (width 0.25) (layer F.Cu) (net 1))
 (segment (start 129.827797 68.94199) (end 137.34599 68.94199) (width 0.25) (layer F.Cu) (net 1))
 (segment (start 129.214 69.555787) (end 129.827797 68.94199) (width 0.25) (layer F.Cu) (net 1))
 (segment (start 129.214 70.97) (end 129.214 69.555787) (width 0.25) (layer F.Cu) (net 1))
 (segment (start 116.84 79.756) (end 114.554 77.47) (width 0.25) (layer F.Cu) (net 3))
 (segment (start 116.84 81.28) (end 116.84 79.756) (width 0.25) (layer F.Cu) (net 3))
 (segment (start 114.554 70.97) (end 114.554 77.47) (width 0.25) (layer F.Cu) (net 3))
 (segment (start 119.013 74.93) (end 119.126 75.043) (width 0.25) (layer B.Cu) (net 3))
 (segment (start 116.445 74.93) (end 119.013 74.93) (width 0.25) (layer B.Cu) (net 3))
 (segment (start 114.921 73.406) (end 116.445 74.93) (width 0.25) (layer B.Cu) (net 3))
 (segment (start 114.695 73.406) (end 114.921 73.406) (width 0.25) (layer B.Cu) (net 3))
 (segment (start 114.695 71.111) (end 114.554 70.97) (width 0.25) (layer B.Cu) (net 3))
 (segment (start 114.695 73.406) (end 114.695 71.111) (width 0.25) (layer B.Cu) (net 3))
 (segment (start 127 79.756) (end 124.714 77.47) (width 0.25) (layer F.Cu) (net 4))
 (segment (start 127 81.28) (end 127 79.756) (width 0.25) (layer F.Cu) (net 4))
 (segment (start 124.714 70.97) (end 124.714 77.47) (width 0.25) (layer F.Cu) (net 4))
 (segment (start 129.173 74.93) (end 129.286 75.043) (width 0.25) (layer B.Cu) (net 4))
 (segment (start 126.351 74.93) (end 129.173 74.93) (width 0.25) (layer B.Cu) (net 4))
 (segment (start 124.827 73.406) (end 126.351 74.93) (width 0.25) (layer B.Cu) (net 4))
 (segment (start 124.601 73.406) (end 124.827 73.406) (width 0.25) (layer B.Cu) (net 4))
 (segment (start 124.601 71.083) (end 124.714 70.97) (width 0.25) (layer B.Cu) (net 4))
 (segment (start 124.601 73.406) (end 124.601 71.083) (width 0.25) (layer B.Cu) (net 4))
 (segment (start 137.16 79.756) (end 134.874 77.47) (width 0.25) (layer F.Cu) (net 5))
 (segment (start 137.16 81.28) (end 137.16 79.756) (width 0.25) (layer F.Cu) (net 5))
 (segment (start 134.874 70.97) (end 134.874 77.47) (width 0.25) (layer F.Cu) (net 5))
 (segment (start 139.333 74.93) (end 139.446 75.043) (width 0.25) (layer B.Cu) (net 5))
 (segment (start 136.511 74.93) (end 139.333 74.93) (width 0.25) (layer B.Cu) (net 5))
 (segment (start 134.987 73.406) (end 136.511 74.93) (width 0.25) (layer B.Cu) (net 5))
 (segment (start 134.761 73.406) (end 134.987 73.406) (width 0.25) (layer B.Cu) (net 5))
 (segment (start 134.761 71.083) (end 134.874 70.97) (width 0.25) (layer B.Cu) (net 5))
 (segment (start 134.761 73.406) (end 134.761 71.083) (width 0.25) (layer B.Cu) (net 5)))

